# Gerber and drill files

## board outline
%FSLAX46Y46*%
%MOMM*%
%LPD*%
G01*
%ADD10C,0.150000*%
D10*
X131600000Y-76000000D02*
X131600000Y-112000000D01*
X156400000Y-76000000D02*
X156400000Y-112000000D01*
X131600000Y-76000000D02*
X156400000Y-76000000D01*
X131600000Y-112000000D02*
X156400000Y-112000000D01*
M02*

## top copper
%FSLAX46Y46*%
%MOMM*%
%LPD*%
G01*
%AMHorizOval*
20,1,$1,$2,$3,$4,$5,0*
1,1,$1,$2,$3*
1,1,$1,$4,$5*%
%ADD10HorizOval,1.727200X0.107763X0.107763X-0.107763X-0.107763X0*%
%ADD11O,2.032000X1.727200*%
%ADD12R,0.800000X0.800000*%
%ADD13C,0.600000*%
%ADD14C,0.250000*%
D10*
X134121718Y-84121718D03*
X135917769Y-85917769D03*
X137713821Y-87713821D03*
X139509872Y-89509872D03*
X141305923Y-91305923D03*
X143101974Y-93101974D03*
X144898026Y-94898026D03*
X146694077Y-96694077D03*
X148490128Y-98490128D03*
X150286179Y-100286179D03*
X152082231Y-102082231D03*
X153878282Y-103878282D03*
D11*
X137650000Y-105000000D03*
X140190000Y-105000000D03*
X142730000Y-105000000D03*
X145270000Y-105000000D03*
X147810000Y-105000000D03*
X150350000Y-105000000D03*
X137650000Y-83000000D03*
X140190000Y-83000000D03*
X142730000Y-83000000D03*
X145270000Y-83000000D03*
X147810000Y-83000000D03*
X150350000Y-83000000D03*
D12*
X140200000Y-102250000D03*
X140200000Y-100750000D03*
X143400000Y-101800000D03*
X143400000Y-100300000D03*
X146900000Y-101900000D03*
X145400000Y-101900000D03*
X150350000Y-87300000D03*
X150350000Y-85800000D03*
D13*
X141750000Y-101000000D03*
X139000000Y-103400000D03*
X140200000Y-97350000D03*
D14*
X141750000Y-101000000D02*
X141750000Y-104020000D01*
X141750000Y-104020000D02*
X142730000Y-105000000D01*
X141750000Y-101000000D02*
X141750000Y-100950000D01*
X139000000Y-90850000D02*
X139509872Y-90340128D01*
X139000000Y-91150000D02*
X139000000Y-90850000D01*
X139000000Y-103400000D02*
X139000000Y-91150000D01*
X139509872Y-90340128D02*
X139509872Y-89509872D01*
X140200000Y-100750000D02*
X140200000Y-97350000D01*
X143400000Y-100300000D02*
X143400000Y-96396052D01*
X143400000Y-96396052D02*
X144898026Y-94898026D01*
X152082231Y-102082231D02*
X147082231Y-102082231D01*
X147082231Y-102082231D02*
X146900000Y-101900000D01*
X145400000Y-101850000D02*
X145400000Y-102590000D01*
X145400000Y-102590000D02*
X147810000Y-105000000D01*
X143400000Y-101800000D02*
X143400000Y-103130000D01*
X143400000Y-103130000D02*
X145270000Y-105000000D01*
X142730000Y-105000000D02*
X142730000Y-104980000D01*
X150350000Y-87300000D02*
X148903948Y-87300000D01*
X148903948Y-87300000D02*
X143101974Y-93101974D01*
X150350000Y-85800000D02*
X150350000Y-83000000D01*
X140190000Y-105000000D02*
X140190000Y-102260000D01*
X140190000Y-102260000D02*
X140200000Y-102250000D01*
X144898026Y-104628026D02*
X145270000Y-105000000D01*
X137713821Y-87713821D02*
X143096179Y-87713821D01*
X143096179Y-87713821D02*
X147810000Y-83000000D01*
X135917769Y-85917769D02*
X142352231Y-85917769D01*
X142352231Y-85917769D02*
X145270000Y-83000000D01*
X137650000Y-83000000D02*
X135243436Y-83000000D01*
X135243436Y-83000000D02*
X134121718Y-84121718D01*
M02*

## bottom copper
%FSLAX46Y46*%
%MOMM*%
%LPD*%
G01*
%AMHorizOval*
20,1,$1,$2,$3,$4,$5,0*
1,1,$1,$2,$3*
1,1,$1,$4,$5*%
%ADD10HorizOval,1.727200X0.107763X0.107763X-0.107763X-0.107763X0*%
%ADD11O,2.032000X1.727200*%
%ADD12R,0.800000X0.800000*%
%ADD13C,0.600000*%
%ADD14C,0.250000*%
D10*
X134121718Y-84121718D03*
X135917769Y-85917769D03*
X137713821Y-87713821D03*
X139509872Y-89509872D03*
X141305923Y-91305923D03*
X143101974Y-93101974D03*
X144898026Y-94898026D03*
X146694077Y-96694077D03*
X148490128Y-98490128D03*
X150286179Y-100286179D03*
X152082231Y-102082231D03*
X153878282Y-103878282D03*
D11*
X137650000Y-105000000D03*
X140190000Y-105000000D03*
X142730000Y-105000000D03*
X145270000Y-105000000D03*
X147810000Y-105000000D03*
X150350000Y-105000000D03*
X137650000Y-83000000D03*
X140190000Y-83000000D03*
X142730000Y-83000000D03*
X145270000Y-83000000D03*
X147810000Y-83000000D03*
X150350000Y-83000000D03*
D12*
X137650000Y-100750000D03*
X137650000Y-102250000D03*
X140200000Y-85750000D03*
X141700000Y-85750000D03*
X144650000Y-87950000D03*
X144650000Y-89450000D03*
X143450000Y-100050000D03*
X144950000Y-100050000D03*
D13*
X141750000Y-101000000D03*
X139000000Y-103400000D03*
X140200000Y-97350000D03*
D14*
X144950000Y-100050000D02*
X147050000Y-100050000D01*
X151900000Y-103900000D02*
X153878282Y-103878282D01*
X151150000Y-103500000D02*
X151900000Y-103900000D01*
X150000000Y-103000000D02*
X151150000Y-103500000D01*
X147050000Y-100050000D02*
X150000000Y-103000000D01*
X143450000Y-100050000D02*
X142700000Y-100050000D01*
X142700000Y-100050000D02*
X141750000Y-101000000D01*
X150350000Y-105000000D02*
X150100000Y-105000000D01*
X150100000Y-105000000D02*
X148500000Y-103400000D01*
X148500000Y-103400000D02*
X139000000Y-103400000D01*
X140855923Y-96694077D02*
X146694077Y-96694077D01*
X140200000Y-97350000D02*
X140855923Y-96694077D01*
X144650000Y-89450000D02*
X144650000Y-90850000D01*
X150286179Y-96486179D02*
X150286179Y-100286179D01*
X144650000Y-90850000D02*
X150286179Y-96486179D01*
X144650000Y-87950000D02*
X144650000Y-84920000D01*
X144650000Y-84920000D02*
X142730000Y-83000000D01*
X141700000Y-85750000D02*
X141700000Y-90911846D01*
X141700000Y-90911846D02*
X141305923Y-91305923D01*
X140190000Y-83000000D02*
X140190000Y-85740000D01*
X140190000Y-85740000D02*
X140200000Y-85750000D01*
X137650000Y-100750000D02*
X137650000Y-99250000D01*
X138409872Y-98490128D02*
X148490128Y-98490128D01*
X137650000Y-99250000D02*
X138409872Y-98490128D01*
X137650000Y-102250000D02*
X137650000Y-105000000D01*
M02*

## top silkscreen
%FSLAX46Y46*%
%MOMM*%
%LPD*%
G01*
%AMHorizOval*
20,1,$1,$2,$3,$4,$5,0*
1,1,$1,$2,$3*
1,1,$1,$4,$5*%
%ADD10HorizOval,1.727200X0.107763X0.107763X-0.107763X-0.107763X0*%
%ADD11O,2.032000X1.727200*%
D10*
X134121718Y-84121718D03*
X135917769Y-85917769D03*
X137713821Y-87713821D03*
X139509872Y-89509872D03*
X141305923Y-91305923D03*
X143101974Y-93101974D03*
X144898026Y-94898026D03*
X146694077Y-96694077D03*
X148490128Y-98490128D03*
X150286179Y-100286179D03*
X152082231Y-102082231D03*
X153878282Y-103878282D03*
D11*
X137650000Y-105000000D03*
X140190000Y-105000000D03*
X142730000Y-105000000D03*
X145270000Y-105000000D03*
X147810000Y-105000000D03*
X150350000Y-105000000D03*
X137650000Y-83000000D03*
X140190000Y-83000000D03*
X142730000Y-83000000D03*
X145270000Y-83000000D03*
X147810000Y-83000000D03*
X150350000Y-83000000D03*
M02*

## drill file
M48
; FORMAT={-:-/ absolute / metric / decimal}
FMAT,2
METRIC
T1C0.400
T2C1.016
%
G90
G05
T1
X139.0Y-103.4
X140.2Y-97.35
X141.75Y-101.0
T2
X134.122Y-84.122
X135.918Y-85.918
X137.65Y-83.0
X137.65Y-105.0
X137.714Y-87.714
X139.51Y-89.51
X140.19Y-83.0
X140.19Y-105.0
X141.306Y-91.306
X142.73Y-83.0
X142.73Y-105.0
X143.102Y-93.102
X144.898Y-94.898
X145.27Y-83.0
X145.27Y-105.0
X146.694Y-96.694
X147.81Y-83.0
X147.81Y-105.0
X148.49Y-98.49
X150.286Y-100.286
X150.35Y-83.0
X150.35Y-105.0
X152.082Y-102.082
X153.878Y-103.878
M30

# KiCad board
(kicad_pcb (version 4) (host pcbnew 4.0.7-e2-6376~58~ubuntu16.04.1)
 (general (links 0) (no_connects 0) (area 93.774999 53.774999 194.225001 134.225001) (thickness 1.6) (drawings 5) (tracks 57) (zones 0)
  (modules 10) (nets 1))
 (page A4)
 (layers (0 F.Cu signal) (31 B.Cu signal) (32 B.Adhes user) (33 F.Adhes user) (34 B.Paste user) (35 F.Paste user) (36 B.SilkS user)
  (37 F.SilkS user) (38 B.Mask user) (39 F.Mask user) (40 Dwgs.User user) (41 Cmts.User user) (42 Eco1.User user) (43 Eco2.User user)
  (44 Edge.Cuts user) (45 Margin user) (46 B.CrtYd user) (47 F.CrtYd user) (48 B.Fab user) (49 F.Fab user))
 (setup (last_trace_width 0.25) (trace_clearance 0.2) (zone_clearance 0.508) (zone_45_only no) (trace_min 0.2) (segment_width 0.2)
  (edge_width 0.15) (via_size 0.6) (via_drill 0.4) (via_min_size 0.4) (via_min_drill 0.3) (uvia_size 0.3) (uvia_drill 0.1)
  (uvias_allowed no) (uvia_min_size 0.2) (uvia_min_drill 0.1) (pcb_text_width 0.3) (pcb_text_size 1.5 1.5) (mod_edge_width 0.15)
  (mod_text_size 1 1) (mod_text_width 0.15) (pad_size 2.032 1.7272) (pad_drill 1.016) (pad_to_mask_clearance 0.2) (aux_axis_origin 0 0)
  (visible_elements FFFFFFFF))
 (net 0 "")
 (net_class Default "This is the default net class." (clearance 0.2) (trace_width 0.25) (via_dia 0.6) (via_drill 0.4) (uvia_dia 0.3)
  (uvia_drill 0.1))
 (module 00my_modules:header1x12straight (layer F.Cu) (at 144 94 45)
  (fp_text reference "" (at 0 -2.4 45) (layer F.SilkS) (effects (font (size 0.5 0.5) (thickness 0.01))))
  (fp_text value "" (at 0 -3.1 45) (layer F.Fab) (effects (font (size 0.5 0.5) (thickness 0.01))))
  (pad 0 thru_hole oval (at 0 -13.97 45) (size 2.032 1.7272) (drill 1.016) (layers *.Cu *.Mask F.SilkS))
  (pad 1 thru_hole oval (at 0 -11.43 45) (size 2.032 1.7272) (drill 1.016) (layers *.Cu *.Mask F.SilkS))
  (pad 2 thru_hole oval (at 0 -8.89 45) (size 2.032 1.7272) (drill 1.016) (layers *.Cu *.Mask F.SilkS))
  (pad 3 thru_hole oval (at 0 -6.35 45) (size 2.032 1.7272) (drill 1.016) (layers *.Cu *.Mask F.SilkS))
  (pad A thru_hole oval (at 0 -3.81 45) (size 2.032 1.7272) (drill 1.016) (layers *.Cu *.Mask F.SilkS))
  (pad B thru_hole oval (at 0 -1.27 45) (size 2.032 1.7272) (drill 1.016) (layers *.Cu *.Mask F.SilkS))
  (pad C thru_hole oval (at 0 1.27 45) (size 2.032 1.7272) (drill 1.016) (layers *.Cu *.Mask F.SilkS))
  (pad D thru_hole oval (at 0 3.81 45) (size 2.032 1.7272) (drill 1.016) (layers *.Cu *.Mask F.SilkS))
  (pad E thru_hole oval (at 0 6.35 45) (size 2.032 1.7272) (drill 1.016) (layers *.Cu *.Mask F.SilkS))
  (pad F thru_hole oval (at 0 8.89 45) (size 2.032 1.7272) (drill 1.016) (layers *.Cu *.Mask F.SilkS))
  (pad G thru_hole oval (at 0 11.43 45) (size 2.032 1.7272) (drill 1.016) (layers *.Cu *.Mask F.SilkS))
  (pad P thru_hole oval (at 0 13.97 45) (size 2.032 1.7272) (drill 1.016) (layers *.Cu *.Mask F.SilkS)))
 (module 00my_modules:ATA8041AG (layer F.Cu) (at 144 94)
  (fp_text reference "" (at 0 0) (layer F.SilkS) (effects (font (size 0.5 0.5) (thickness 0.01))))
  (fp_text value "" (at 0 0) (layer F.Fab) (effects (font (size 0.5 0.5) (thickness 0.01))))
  (pad E thru_hole oval (at -6.35 11) (size 2.032 1.7272) (drill 1.016) (layers *.Cu *.Mask F.SilkS))
  (pad D thru_hole oval (at -3.81 11) (size 2.032 1.7272) (drill 1.016) (layers *.Cu *.Mask F.SilkS))
  (pad P thru_hole oval (at -1.27 11) (size 2.032 1.7272) (drill 1.016) (layers *.Cu *.Mask F.SilkS))
  (pad C thru_hole oval (at 1.27 11) (size 2.032 1.7272) (drill 1.016) (layers *.Cu *.Mask F.SilkS))
  (pad G thru_hole oval (at 3.81 11) (size 2.032 1.7272) (drill 1.016) (layers *.Cu *.Mask F.SilkS))
  (pad 3 thru_hole oval (at 6.35 11) (size 2.032 1.7272) (drill 1.016) (layers *.Cu *.Mask F.SilkS))
  (pad 0 thru_hole oval (at -6.35 -11) (size 2.032 1.7272) (drill 1.016) (layers *.Cu *.Mask F.SilkS))
  (pad A thru_hole oval (at -3.81 -11) (size 2.032 1.7272) (drill 1.016) (layers *.Cu *.Mask F.SilkS))
  (pad F thru_hole oval (at -1.27 -11) (size 2.032 1.7272) (drill 1.016) (layers *.Cu *.Mask F.SilkS))
  (pad 1 thru_hole oval (at 1.27 -11) (size 2.032 1.7272) (drill 1.016) (layers *.Cu *.Mask F.SilkS))
  (pad 2 thru_hole oval (at 3.81 -11) (size 2.032 1.7272) (drill 1.016) (layers *.Cu *.Mask F.SilkS))
  (pad B thru_hole oval (at 6.35 -11) (size 2.032 1.7272) (drill 1.016) (layers *.Cu *.Mask F.SilkS)))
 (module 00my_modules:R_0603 (layer B.Cu) (at 137.65 101.5 270)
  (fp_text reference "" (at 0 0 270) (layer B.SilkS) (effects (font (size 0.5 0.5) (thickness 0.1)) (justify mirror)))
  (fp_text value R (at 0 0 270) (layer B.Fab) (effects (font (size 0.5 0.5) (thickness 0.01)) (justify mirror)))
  (pad 1 smd rect (at -0.75 0 270) (size 0.8 0.8) (layers B.Cu B.Paste B.Mask))
  (pad 2 smd rect (at 0.75 0 270) (size 0.8 0.8) (layers B.Cu B.Paste B.Mask)))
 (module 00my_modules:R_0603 (layer F.Cu) (at 140.2 101.5 90)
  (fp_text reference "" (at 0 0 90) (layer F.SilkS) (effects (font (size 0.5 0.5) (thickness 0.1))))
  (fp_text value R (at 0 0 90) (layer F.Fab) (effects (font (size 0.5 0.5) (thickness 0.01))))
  (pad 1 smd rect (at -0.75 0 90) (size 0.8 0.8) (layers F.Cu F.Paste F.Mask))
  (pad 2 smd rect (at 0.75 0 90) (size 0.8 0.8) (layers F.Cu F.Paste F.Mask)))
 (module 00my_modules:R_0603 (layer F.Cu) (at 143.4 101.05 90)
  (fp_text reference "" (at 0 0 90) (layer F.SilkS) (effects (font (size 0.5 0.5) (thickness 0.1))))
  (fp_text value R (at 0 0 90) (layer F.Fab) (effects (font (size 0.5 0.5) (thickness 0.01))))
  (pad 1 smd rect (at -0.75 0 90) (size 0.8 0.8) (layers F.Cu F.Paste F.Mask))
  (pad 2 smd rect (at 0.75 0 90) (size 0.8 0.8) (layers F.Cu F.Paste F.Mask)))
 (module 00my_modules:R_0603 (layer F.Cu) (at 146.15 101.9 180)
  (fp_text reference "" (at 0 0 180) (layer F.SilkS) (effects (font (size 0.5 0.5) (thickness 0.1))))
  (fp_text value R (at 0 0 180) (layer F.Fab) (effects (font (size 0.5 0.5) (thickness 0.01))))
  (pad 1 smd rect (at -0.75 0 180) (size 0.8 0.8) (layers F.Cu F.Paste F.Mask))
  (pad 2 smd rect (at 0.75 0 180) (size 0.8 0.8) (layers F.Cu F.Paste F.Mask)))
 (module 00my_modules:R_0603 (layer B.Cu) (at 140.95 85.75)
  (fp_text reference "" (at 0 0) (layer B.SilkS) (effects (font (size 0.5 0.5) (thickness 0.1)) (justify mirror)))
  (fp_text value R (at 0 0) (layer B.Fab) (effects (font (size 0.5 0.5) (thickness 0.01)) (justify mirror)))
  (pad 1 smd rect (at -0.75 0) (size 0.8 0.8) (layers B.Cu B.Paste B.Mask))
  (pad 2 smd rect (at 0.75 0) (size 0.8 0.8) (layers B.Cu B.Paste B.Mask)))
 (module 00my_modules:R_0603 (layer B.Cu) (at 144.65 88.7 270)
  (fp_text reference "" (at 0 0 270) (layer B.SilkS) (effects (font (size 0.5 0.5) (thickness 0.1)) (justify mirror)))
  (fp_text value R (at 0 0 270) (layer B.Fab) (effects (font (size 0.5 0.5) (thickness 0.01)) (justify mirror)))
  (pad 1 smd rect (at -0.75 0 270) (size 0.8 0.8) (layers B.Cu B.Paste B.Mask))
  (pad 2 smd rect (at 0.75 0 270) (size 0.8 0.8) (layers B.Cu B.Paste B.Mask)))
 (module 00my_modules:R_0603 (layer F.Cu) (at 150.35 86.55 90)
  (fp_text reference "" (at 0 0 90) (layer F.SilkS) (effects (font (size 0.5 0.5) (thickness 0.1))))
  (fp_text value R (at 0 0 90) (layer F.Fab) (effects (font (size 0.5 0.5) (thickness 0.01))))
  (pad 1 smd rect (at -0.75 0 90) (size 0.8 0.8) (layers F.Cu F.Paste F.Mask))
  (pad 2 smd rect (at 0.75 0 90) (size 0.8 0.8) (layers F.Cu F.Paste F.Mask)))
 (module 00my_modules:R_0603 (layer B.Cu) (at 144.2 100.05)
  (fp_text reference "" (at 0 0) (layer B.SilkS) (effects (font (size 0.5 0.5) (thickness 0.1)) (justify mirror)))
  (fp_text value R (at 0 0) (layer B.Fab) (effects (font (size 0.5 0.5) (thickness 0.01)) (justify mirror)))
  (pad 1 smd rect (at -0.75 0) (size 0.8 0.8) (layers B.Cu B.Paste B.Mask))
  (pad 2 smd rect (at 0.75 0) (size 0.8 0.8) (layers B.Cu B.Paste B.Mask)))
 (gr_line (start 131.6 76) (end 131.6 112) (angle 90) (layer Edge.Cuts) (width 0.15))
 (gr_line (start 156.4 76) (end 156.4 112) (angle 90) (layer Edge.Cuts) (width 0.15))
 (gr_line (start 131.6 76) (end 156.4 76) (angle 90) (layer Edge.Cuts) (width 0.15))
 (gr_line (start 131.6 112) (end 156.4 112) (angle 90) (layer Edge.Cuts) (width 0.15))
 (segment (start 144.95 100.05) (end 147.05 100.05) (width 0.25) (layer B.Cu) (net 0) (status 400000))
 (segment (start 151.9 103.9) (end 153.878282 103.878282) (width 0.25) (layer B.Cu) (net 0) (status 800000))
 (segment (start 151.15 103.5) (end 151.9 103.9) (width 0.25) (layer B.Cu) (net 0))
 (segment (start 150 103) (end 151.15 103.5) (width 0.25) (layer B.Cu) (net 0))
 (segment (start 147.05 100.05) (end 150 103) (width 0.25) (layer B.Cu) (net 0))
 (segment (start 141.75 101) (end 141.75 104.02) (width 0.25) (layer F.Cu) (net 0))
 (segment (start 141.75 104.02) (end 142.73 105) (width 0.25) (layer F.Cu) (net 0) (status 800000))
 (segment (start 143.45 100.05) (end 142.7 100.05) (width 0.25) (layer B.Cu) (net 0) (status 400000))
 (segment (start 141.75 101) (end 141.75 100.95) (width 0.25) (layer F.Cu) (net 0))
 (via (at 141.75 101) (size 0.6) (drill 0.4) (layers F.Cu B.Cu) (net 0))
 (segment (start 142.7 100.05) (end 141.75 101) (width 0.25) (layer B.Cu) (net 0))
 (segment (start 150.35 105) (end 150.1 105) (width 0.25) (layer B.Cu) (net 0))
 (segment (start 150.1 105) (end 148.5 103.4) (width 0.25) (layer B.Cu) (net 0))
 (segment (start 139 90.85) (end 139.509872 90.340128) (width 0.25) (layer F.Cu) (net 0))
 (segment (start 139 91.15) (end 139 90.85) (width 0.25) (layer F.Cu) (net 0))
 (segment (start 139 103.4) (end 139 91.15) (width 0.25) (layer F.Cu) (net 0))
 (via (at 139 103.4) (size 0.6) (drill 0.4) (layers F.Cu B.Cu) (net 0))
 (segment (start 148.5 103.4) (end 139 103.4) (width 0.25) (layer B.Cu) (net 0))
 (segment (start 139.509872 90.340128) (end 139.509872 89.509872) (width 0.25) (layer F.Cu) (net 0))
 (segment (start 140.2 100.75) (end 140.2 97.35) (width 0.25) (layer F.Cu) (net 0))
 (segment (start 140.855923 96.694077) (end 146.694077 96.694077) (width 0.25) (layer B.Cu) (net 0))
 (segment (start 140.2 97.35) (end 140.855923 96.694077) (width 0.25) (layer B.Cu) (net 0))
 (via (at 140.2 97.35) (size 0.6) (drill 0.4) (layers F.Cu B.Cu) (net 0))
 (segment (start 143.4 100.3) (end 143.4 96.396052) (width 0.25) (layer F.Cu) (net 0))
 (segment (start 143.4 96.396052) (end 144.898026 94.898026) (width 0.25) (layer F.Cu) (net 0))
 (segment (start 152.082231 102.082231) (end 147.082231 102.082231) (width 0.25) (layer F.Cu) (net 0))
 (segment (start 147.082231 102.082231) (end 146.9 101.9) (width 0.25) (layer F.Cu) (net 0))
 (segment (start 145.4 101.85) (end 145.4 102.59) (width 0.25) (layer F.Cu) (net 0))
 (segment (start 145.4 102.59) (end 147.81 105) (width 0.25) (layer F.Cu) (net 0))
 (segment (start 143.4 101.8) (end 143.4 103.13) (width 0.25) (layer F.Cu) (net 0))
 (segment (start 143.4 103.13) (end 145.27 105) (width 0.25) (layer F.Cu) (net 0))
 (segment (start 142.73 105) (end 142.73 104.98) (width 0.25) (layer F.Cu) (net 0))
 (segment (start 144.65 89.45) (end 144.65 90.85) (width 0.25) (layer B.Cu) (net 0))
 (segment (start 150.286179 96.486179) (end 150.286179 100.286179) (width 0.25) (layer B.Cu) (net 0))
 (segment (start 144.65 90.85) (end 150.286179 96.486179) (width 0.25) (layer B.Cu) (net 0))
 (segment (start 144.65 87.95) (end 144.65 84.92) (width 0.25) (layer B.Cu) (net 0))
 (segment (start 144.65 84.92) (end 142.73 83) (width 0.25) (layer B.Cu) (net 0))
 (segment (start 150.35 87.3) (end 148.903948 87.3) (width 0.25) (layer F.Cu) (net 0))
 (segment (start 148.903948 87.3) (end 143.101974 93.101974) (width 0.25) (layer F.Cu) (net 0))
 (segment (start 150.35 85.8) (end 150.35 83) (width 0.25) (layer F.Cu) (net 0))
 (segment (start 141.7 85.75) (end 141.7 90.911846) (width 0.25) (layer B.Cu) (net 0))
 (segment (start 141.7 90.911846) (end 141.305923 91.305923) (width 0.25) (layer B.Cu) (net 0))
 (segment (start 140.19 83) (end 140.19 85.74) (width 0.25) (layer B.Cu) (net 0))
 (segment (start 140.19 85.74) (end 140.2 85.75) (width 0.25) (layer B.Cu) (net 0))
 (segment (start 140.19 105) (end 140.19 102.26) (width 0.25) (layer F.Cu) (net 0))
 (segment (start 140.19 102.26) (end 140.2 102.25) (width 0.25) (layer F.Cu) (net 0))
 (segment (start 137.65 100.75) (end 137.65 99.25) (width 0.25) (layer B.Cu) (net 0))
 (segment (start 138.409872 98.490128) (end 148.490128 98.490128) (width 0.25) (layer B.Cu) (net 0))
 (segment (start 137.65 99.25) (end 138.409872 98.490128) (width 0.25) (layer B.Cu) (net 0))
 (segment (start 137.65 102.25) (end 137.65 105) (width 0.25) (layer B.Cu) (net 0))
 (segment (start 144.898026 104.628026) (end 145.27 105) (width 0.25) (layer F.Cu) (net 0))
 (segment (start 137.713821 87.713821) (end 143.096179 87.713821) (width 0.25) (layer F.Cu) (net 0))
 (segment (start 143.096179 87.713821) (end 147.81 83) (width 0.25) (layer F.Cu) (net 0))
 (segment (start 135.917769 85.917769) (end 142.352231 85.917769) (width 0.25) (layer F.Cu) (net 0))
 (segment (start 142.352231 85.917769) (end 145.27 83) (width 0.25) (layer F.Cu) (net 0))
 (segment (start 137.65 83) (end 135.243436 83) (width 0.25) (layer F.Cu) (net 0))
 (segment (start 135.243436 83) (end 134.121718 84.121718) (width 0.25) (layer F.Cu) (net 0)))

